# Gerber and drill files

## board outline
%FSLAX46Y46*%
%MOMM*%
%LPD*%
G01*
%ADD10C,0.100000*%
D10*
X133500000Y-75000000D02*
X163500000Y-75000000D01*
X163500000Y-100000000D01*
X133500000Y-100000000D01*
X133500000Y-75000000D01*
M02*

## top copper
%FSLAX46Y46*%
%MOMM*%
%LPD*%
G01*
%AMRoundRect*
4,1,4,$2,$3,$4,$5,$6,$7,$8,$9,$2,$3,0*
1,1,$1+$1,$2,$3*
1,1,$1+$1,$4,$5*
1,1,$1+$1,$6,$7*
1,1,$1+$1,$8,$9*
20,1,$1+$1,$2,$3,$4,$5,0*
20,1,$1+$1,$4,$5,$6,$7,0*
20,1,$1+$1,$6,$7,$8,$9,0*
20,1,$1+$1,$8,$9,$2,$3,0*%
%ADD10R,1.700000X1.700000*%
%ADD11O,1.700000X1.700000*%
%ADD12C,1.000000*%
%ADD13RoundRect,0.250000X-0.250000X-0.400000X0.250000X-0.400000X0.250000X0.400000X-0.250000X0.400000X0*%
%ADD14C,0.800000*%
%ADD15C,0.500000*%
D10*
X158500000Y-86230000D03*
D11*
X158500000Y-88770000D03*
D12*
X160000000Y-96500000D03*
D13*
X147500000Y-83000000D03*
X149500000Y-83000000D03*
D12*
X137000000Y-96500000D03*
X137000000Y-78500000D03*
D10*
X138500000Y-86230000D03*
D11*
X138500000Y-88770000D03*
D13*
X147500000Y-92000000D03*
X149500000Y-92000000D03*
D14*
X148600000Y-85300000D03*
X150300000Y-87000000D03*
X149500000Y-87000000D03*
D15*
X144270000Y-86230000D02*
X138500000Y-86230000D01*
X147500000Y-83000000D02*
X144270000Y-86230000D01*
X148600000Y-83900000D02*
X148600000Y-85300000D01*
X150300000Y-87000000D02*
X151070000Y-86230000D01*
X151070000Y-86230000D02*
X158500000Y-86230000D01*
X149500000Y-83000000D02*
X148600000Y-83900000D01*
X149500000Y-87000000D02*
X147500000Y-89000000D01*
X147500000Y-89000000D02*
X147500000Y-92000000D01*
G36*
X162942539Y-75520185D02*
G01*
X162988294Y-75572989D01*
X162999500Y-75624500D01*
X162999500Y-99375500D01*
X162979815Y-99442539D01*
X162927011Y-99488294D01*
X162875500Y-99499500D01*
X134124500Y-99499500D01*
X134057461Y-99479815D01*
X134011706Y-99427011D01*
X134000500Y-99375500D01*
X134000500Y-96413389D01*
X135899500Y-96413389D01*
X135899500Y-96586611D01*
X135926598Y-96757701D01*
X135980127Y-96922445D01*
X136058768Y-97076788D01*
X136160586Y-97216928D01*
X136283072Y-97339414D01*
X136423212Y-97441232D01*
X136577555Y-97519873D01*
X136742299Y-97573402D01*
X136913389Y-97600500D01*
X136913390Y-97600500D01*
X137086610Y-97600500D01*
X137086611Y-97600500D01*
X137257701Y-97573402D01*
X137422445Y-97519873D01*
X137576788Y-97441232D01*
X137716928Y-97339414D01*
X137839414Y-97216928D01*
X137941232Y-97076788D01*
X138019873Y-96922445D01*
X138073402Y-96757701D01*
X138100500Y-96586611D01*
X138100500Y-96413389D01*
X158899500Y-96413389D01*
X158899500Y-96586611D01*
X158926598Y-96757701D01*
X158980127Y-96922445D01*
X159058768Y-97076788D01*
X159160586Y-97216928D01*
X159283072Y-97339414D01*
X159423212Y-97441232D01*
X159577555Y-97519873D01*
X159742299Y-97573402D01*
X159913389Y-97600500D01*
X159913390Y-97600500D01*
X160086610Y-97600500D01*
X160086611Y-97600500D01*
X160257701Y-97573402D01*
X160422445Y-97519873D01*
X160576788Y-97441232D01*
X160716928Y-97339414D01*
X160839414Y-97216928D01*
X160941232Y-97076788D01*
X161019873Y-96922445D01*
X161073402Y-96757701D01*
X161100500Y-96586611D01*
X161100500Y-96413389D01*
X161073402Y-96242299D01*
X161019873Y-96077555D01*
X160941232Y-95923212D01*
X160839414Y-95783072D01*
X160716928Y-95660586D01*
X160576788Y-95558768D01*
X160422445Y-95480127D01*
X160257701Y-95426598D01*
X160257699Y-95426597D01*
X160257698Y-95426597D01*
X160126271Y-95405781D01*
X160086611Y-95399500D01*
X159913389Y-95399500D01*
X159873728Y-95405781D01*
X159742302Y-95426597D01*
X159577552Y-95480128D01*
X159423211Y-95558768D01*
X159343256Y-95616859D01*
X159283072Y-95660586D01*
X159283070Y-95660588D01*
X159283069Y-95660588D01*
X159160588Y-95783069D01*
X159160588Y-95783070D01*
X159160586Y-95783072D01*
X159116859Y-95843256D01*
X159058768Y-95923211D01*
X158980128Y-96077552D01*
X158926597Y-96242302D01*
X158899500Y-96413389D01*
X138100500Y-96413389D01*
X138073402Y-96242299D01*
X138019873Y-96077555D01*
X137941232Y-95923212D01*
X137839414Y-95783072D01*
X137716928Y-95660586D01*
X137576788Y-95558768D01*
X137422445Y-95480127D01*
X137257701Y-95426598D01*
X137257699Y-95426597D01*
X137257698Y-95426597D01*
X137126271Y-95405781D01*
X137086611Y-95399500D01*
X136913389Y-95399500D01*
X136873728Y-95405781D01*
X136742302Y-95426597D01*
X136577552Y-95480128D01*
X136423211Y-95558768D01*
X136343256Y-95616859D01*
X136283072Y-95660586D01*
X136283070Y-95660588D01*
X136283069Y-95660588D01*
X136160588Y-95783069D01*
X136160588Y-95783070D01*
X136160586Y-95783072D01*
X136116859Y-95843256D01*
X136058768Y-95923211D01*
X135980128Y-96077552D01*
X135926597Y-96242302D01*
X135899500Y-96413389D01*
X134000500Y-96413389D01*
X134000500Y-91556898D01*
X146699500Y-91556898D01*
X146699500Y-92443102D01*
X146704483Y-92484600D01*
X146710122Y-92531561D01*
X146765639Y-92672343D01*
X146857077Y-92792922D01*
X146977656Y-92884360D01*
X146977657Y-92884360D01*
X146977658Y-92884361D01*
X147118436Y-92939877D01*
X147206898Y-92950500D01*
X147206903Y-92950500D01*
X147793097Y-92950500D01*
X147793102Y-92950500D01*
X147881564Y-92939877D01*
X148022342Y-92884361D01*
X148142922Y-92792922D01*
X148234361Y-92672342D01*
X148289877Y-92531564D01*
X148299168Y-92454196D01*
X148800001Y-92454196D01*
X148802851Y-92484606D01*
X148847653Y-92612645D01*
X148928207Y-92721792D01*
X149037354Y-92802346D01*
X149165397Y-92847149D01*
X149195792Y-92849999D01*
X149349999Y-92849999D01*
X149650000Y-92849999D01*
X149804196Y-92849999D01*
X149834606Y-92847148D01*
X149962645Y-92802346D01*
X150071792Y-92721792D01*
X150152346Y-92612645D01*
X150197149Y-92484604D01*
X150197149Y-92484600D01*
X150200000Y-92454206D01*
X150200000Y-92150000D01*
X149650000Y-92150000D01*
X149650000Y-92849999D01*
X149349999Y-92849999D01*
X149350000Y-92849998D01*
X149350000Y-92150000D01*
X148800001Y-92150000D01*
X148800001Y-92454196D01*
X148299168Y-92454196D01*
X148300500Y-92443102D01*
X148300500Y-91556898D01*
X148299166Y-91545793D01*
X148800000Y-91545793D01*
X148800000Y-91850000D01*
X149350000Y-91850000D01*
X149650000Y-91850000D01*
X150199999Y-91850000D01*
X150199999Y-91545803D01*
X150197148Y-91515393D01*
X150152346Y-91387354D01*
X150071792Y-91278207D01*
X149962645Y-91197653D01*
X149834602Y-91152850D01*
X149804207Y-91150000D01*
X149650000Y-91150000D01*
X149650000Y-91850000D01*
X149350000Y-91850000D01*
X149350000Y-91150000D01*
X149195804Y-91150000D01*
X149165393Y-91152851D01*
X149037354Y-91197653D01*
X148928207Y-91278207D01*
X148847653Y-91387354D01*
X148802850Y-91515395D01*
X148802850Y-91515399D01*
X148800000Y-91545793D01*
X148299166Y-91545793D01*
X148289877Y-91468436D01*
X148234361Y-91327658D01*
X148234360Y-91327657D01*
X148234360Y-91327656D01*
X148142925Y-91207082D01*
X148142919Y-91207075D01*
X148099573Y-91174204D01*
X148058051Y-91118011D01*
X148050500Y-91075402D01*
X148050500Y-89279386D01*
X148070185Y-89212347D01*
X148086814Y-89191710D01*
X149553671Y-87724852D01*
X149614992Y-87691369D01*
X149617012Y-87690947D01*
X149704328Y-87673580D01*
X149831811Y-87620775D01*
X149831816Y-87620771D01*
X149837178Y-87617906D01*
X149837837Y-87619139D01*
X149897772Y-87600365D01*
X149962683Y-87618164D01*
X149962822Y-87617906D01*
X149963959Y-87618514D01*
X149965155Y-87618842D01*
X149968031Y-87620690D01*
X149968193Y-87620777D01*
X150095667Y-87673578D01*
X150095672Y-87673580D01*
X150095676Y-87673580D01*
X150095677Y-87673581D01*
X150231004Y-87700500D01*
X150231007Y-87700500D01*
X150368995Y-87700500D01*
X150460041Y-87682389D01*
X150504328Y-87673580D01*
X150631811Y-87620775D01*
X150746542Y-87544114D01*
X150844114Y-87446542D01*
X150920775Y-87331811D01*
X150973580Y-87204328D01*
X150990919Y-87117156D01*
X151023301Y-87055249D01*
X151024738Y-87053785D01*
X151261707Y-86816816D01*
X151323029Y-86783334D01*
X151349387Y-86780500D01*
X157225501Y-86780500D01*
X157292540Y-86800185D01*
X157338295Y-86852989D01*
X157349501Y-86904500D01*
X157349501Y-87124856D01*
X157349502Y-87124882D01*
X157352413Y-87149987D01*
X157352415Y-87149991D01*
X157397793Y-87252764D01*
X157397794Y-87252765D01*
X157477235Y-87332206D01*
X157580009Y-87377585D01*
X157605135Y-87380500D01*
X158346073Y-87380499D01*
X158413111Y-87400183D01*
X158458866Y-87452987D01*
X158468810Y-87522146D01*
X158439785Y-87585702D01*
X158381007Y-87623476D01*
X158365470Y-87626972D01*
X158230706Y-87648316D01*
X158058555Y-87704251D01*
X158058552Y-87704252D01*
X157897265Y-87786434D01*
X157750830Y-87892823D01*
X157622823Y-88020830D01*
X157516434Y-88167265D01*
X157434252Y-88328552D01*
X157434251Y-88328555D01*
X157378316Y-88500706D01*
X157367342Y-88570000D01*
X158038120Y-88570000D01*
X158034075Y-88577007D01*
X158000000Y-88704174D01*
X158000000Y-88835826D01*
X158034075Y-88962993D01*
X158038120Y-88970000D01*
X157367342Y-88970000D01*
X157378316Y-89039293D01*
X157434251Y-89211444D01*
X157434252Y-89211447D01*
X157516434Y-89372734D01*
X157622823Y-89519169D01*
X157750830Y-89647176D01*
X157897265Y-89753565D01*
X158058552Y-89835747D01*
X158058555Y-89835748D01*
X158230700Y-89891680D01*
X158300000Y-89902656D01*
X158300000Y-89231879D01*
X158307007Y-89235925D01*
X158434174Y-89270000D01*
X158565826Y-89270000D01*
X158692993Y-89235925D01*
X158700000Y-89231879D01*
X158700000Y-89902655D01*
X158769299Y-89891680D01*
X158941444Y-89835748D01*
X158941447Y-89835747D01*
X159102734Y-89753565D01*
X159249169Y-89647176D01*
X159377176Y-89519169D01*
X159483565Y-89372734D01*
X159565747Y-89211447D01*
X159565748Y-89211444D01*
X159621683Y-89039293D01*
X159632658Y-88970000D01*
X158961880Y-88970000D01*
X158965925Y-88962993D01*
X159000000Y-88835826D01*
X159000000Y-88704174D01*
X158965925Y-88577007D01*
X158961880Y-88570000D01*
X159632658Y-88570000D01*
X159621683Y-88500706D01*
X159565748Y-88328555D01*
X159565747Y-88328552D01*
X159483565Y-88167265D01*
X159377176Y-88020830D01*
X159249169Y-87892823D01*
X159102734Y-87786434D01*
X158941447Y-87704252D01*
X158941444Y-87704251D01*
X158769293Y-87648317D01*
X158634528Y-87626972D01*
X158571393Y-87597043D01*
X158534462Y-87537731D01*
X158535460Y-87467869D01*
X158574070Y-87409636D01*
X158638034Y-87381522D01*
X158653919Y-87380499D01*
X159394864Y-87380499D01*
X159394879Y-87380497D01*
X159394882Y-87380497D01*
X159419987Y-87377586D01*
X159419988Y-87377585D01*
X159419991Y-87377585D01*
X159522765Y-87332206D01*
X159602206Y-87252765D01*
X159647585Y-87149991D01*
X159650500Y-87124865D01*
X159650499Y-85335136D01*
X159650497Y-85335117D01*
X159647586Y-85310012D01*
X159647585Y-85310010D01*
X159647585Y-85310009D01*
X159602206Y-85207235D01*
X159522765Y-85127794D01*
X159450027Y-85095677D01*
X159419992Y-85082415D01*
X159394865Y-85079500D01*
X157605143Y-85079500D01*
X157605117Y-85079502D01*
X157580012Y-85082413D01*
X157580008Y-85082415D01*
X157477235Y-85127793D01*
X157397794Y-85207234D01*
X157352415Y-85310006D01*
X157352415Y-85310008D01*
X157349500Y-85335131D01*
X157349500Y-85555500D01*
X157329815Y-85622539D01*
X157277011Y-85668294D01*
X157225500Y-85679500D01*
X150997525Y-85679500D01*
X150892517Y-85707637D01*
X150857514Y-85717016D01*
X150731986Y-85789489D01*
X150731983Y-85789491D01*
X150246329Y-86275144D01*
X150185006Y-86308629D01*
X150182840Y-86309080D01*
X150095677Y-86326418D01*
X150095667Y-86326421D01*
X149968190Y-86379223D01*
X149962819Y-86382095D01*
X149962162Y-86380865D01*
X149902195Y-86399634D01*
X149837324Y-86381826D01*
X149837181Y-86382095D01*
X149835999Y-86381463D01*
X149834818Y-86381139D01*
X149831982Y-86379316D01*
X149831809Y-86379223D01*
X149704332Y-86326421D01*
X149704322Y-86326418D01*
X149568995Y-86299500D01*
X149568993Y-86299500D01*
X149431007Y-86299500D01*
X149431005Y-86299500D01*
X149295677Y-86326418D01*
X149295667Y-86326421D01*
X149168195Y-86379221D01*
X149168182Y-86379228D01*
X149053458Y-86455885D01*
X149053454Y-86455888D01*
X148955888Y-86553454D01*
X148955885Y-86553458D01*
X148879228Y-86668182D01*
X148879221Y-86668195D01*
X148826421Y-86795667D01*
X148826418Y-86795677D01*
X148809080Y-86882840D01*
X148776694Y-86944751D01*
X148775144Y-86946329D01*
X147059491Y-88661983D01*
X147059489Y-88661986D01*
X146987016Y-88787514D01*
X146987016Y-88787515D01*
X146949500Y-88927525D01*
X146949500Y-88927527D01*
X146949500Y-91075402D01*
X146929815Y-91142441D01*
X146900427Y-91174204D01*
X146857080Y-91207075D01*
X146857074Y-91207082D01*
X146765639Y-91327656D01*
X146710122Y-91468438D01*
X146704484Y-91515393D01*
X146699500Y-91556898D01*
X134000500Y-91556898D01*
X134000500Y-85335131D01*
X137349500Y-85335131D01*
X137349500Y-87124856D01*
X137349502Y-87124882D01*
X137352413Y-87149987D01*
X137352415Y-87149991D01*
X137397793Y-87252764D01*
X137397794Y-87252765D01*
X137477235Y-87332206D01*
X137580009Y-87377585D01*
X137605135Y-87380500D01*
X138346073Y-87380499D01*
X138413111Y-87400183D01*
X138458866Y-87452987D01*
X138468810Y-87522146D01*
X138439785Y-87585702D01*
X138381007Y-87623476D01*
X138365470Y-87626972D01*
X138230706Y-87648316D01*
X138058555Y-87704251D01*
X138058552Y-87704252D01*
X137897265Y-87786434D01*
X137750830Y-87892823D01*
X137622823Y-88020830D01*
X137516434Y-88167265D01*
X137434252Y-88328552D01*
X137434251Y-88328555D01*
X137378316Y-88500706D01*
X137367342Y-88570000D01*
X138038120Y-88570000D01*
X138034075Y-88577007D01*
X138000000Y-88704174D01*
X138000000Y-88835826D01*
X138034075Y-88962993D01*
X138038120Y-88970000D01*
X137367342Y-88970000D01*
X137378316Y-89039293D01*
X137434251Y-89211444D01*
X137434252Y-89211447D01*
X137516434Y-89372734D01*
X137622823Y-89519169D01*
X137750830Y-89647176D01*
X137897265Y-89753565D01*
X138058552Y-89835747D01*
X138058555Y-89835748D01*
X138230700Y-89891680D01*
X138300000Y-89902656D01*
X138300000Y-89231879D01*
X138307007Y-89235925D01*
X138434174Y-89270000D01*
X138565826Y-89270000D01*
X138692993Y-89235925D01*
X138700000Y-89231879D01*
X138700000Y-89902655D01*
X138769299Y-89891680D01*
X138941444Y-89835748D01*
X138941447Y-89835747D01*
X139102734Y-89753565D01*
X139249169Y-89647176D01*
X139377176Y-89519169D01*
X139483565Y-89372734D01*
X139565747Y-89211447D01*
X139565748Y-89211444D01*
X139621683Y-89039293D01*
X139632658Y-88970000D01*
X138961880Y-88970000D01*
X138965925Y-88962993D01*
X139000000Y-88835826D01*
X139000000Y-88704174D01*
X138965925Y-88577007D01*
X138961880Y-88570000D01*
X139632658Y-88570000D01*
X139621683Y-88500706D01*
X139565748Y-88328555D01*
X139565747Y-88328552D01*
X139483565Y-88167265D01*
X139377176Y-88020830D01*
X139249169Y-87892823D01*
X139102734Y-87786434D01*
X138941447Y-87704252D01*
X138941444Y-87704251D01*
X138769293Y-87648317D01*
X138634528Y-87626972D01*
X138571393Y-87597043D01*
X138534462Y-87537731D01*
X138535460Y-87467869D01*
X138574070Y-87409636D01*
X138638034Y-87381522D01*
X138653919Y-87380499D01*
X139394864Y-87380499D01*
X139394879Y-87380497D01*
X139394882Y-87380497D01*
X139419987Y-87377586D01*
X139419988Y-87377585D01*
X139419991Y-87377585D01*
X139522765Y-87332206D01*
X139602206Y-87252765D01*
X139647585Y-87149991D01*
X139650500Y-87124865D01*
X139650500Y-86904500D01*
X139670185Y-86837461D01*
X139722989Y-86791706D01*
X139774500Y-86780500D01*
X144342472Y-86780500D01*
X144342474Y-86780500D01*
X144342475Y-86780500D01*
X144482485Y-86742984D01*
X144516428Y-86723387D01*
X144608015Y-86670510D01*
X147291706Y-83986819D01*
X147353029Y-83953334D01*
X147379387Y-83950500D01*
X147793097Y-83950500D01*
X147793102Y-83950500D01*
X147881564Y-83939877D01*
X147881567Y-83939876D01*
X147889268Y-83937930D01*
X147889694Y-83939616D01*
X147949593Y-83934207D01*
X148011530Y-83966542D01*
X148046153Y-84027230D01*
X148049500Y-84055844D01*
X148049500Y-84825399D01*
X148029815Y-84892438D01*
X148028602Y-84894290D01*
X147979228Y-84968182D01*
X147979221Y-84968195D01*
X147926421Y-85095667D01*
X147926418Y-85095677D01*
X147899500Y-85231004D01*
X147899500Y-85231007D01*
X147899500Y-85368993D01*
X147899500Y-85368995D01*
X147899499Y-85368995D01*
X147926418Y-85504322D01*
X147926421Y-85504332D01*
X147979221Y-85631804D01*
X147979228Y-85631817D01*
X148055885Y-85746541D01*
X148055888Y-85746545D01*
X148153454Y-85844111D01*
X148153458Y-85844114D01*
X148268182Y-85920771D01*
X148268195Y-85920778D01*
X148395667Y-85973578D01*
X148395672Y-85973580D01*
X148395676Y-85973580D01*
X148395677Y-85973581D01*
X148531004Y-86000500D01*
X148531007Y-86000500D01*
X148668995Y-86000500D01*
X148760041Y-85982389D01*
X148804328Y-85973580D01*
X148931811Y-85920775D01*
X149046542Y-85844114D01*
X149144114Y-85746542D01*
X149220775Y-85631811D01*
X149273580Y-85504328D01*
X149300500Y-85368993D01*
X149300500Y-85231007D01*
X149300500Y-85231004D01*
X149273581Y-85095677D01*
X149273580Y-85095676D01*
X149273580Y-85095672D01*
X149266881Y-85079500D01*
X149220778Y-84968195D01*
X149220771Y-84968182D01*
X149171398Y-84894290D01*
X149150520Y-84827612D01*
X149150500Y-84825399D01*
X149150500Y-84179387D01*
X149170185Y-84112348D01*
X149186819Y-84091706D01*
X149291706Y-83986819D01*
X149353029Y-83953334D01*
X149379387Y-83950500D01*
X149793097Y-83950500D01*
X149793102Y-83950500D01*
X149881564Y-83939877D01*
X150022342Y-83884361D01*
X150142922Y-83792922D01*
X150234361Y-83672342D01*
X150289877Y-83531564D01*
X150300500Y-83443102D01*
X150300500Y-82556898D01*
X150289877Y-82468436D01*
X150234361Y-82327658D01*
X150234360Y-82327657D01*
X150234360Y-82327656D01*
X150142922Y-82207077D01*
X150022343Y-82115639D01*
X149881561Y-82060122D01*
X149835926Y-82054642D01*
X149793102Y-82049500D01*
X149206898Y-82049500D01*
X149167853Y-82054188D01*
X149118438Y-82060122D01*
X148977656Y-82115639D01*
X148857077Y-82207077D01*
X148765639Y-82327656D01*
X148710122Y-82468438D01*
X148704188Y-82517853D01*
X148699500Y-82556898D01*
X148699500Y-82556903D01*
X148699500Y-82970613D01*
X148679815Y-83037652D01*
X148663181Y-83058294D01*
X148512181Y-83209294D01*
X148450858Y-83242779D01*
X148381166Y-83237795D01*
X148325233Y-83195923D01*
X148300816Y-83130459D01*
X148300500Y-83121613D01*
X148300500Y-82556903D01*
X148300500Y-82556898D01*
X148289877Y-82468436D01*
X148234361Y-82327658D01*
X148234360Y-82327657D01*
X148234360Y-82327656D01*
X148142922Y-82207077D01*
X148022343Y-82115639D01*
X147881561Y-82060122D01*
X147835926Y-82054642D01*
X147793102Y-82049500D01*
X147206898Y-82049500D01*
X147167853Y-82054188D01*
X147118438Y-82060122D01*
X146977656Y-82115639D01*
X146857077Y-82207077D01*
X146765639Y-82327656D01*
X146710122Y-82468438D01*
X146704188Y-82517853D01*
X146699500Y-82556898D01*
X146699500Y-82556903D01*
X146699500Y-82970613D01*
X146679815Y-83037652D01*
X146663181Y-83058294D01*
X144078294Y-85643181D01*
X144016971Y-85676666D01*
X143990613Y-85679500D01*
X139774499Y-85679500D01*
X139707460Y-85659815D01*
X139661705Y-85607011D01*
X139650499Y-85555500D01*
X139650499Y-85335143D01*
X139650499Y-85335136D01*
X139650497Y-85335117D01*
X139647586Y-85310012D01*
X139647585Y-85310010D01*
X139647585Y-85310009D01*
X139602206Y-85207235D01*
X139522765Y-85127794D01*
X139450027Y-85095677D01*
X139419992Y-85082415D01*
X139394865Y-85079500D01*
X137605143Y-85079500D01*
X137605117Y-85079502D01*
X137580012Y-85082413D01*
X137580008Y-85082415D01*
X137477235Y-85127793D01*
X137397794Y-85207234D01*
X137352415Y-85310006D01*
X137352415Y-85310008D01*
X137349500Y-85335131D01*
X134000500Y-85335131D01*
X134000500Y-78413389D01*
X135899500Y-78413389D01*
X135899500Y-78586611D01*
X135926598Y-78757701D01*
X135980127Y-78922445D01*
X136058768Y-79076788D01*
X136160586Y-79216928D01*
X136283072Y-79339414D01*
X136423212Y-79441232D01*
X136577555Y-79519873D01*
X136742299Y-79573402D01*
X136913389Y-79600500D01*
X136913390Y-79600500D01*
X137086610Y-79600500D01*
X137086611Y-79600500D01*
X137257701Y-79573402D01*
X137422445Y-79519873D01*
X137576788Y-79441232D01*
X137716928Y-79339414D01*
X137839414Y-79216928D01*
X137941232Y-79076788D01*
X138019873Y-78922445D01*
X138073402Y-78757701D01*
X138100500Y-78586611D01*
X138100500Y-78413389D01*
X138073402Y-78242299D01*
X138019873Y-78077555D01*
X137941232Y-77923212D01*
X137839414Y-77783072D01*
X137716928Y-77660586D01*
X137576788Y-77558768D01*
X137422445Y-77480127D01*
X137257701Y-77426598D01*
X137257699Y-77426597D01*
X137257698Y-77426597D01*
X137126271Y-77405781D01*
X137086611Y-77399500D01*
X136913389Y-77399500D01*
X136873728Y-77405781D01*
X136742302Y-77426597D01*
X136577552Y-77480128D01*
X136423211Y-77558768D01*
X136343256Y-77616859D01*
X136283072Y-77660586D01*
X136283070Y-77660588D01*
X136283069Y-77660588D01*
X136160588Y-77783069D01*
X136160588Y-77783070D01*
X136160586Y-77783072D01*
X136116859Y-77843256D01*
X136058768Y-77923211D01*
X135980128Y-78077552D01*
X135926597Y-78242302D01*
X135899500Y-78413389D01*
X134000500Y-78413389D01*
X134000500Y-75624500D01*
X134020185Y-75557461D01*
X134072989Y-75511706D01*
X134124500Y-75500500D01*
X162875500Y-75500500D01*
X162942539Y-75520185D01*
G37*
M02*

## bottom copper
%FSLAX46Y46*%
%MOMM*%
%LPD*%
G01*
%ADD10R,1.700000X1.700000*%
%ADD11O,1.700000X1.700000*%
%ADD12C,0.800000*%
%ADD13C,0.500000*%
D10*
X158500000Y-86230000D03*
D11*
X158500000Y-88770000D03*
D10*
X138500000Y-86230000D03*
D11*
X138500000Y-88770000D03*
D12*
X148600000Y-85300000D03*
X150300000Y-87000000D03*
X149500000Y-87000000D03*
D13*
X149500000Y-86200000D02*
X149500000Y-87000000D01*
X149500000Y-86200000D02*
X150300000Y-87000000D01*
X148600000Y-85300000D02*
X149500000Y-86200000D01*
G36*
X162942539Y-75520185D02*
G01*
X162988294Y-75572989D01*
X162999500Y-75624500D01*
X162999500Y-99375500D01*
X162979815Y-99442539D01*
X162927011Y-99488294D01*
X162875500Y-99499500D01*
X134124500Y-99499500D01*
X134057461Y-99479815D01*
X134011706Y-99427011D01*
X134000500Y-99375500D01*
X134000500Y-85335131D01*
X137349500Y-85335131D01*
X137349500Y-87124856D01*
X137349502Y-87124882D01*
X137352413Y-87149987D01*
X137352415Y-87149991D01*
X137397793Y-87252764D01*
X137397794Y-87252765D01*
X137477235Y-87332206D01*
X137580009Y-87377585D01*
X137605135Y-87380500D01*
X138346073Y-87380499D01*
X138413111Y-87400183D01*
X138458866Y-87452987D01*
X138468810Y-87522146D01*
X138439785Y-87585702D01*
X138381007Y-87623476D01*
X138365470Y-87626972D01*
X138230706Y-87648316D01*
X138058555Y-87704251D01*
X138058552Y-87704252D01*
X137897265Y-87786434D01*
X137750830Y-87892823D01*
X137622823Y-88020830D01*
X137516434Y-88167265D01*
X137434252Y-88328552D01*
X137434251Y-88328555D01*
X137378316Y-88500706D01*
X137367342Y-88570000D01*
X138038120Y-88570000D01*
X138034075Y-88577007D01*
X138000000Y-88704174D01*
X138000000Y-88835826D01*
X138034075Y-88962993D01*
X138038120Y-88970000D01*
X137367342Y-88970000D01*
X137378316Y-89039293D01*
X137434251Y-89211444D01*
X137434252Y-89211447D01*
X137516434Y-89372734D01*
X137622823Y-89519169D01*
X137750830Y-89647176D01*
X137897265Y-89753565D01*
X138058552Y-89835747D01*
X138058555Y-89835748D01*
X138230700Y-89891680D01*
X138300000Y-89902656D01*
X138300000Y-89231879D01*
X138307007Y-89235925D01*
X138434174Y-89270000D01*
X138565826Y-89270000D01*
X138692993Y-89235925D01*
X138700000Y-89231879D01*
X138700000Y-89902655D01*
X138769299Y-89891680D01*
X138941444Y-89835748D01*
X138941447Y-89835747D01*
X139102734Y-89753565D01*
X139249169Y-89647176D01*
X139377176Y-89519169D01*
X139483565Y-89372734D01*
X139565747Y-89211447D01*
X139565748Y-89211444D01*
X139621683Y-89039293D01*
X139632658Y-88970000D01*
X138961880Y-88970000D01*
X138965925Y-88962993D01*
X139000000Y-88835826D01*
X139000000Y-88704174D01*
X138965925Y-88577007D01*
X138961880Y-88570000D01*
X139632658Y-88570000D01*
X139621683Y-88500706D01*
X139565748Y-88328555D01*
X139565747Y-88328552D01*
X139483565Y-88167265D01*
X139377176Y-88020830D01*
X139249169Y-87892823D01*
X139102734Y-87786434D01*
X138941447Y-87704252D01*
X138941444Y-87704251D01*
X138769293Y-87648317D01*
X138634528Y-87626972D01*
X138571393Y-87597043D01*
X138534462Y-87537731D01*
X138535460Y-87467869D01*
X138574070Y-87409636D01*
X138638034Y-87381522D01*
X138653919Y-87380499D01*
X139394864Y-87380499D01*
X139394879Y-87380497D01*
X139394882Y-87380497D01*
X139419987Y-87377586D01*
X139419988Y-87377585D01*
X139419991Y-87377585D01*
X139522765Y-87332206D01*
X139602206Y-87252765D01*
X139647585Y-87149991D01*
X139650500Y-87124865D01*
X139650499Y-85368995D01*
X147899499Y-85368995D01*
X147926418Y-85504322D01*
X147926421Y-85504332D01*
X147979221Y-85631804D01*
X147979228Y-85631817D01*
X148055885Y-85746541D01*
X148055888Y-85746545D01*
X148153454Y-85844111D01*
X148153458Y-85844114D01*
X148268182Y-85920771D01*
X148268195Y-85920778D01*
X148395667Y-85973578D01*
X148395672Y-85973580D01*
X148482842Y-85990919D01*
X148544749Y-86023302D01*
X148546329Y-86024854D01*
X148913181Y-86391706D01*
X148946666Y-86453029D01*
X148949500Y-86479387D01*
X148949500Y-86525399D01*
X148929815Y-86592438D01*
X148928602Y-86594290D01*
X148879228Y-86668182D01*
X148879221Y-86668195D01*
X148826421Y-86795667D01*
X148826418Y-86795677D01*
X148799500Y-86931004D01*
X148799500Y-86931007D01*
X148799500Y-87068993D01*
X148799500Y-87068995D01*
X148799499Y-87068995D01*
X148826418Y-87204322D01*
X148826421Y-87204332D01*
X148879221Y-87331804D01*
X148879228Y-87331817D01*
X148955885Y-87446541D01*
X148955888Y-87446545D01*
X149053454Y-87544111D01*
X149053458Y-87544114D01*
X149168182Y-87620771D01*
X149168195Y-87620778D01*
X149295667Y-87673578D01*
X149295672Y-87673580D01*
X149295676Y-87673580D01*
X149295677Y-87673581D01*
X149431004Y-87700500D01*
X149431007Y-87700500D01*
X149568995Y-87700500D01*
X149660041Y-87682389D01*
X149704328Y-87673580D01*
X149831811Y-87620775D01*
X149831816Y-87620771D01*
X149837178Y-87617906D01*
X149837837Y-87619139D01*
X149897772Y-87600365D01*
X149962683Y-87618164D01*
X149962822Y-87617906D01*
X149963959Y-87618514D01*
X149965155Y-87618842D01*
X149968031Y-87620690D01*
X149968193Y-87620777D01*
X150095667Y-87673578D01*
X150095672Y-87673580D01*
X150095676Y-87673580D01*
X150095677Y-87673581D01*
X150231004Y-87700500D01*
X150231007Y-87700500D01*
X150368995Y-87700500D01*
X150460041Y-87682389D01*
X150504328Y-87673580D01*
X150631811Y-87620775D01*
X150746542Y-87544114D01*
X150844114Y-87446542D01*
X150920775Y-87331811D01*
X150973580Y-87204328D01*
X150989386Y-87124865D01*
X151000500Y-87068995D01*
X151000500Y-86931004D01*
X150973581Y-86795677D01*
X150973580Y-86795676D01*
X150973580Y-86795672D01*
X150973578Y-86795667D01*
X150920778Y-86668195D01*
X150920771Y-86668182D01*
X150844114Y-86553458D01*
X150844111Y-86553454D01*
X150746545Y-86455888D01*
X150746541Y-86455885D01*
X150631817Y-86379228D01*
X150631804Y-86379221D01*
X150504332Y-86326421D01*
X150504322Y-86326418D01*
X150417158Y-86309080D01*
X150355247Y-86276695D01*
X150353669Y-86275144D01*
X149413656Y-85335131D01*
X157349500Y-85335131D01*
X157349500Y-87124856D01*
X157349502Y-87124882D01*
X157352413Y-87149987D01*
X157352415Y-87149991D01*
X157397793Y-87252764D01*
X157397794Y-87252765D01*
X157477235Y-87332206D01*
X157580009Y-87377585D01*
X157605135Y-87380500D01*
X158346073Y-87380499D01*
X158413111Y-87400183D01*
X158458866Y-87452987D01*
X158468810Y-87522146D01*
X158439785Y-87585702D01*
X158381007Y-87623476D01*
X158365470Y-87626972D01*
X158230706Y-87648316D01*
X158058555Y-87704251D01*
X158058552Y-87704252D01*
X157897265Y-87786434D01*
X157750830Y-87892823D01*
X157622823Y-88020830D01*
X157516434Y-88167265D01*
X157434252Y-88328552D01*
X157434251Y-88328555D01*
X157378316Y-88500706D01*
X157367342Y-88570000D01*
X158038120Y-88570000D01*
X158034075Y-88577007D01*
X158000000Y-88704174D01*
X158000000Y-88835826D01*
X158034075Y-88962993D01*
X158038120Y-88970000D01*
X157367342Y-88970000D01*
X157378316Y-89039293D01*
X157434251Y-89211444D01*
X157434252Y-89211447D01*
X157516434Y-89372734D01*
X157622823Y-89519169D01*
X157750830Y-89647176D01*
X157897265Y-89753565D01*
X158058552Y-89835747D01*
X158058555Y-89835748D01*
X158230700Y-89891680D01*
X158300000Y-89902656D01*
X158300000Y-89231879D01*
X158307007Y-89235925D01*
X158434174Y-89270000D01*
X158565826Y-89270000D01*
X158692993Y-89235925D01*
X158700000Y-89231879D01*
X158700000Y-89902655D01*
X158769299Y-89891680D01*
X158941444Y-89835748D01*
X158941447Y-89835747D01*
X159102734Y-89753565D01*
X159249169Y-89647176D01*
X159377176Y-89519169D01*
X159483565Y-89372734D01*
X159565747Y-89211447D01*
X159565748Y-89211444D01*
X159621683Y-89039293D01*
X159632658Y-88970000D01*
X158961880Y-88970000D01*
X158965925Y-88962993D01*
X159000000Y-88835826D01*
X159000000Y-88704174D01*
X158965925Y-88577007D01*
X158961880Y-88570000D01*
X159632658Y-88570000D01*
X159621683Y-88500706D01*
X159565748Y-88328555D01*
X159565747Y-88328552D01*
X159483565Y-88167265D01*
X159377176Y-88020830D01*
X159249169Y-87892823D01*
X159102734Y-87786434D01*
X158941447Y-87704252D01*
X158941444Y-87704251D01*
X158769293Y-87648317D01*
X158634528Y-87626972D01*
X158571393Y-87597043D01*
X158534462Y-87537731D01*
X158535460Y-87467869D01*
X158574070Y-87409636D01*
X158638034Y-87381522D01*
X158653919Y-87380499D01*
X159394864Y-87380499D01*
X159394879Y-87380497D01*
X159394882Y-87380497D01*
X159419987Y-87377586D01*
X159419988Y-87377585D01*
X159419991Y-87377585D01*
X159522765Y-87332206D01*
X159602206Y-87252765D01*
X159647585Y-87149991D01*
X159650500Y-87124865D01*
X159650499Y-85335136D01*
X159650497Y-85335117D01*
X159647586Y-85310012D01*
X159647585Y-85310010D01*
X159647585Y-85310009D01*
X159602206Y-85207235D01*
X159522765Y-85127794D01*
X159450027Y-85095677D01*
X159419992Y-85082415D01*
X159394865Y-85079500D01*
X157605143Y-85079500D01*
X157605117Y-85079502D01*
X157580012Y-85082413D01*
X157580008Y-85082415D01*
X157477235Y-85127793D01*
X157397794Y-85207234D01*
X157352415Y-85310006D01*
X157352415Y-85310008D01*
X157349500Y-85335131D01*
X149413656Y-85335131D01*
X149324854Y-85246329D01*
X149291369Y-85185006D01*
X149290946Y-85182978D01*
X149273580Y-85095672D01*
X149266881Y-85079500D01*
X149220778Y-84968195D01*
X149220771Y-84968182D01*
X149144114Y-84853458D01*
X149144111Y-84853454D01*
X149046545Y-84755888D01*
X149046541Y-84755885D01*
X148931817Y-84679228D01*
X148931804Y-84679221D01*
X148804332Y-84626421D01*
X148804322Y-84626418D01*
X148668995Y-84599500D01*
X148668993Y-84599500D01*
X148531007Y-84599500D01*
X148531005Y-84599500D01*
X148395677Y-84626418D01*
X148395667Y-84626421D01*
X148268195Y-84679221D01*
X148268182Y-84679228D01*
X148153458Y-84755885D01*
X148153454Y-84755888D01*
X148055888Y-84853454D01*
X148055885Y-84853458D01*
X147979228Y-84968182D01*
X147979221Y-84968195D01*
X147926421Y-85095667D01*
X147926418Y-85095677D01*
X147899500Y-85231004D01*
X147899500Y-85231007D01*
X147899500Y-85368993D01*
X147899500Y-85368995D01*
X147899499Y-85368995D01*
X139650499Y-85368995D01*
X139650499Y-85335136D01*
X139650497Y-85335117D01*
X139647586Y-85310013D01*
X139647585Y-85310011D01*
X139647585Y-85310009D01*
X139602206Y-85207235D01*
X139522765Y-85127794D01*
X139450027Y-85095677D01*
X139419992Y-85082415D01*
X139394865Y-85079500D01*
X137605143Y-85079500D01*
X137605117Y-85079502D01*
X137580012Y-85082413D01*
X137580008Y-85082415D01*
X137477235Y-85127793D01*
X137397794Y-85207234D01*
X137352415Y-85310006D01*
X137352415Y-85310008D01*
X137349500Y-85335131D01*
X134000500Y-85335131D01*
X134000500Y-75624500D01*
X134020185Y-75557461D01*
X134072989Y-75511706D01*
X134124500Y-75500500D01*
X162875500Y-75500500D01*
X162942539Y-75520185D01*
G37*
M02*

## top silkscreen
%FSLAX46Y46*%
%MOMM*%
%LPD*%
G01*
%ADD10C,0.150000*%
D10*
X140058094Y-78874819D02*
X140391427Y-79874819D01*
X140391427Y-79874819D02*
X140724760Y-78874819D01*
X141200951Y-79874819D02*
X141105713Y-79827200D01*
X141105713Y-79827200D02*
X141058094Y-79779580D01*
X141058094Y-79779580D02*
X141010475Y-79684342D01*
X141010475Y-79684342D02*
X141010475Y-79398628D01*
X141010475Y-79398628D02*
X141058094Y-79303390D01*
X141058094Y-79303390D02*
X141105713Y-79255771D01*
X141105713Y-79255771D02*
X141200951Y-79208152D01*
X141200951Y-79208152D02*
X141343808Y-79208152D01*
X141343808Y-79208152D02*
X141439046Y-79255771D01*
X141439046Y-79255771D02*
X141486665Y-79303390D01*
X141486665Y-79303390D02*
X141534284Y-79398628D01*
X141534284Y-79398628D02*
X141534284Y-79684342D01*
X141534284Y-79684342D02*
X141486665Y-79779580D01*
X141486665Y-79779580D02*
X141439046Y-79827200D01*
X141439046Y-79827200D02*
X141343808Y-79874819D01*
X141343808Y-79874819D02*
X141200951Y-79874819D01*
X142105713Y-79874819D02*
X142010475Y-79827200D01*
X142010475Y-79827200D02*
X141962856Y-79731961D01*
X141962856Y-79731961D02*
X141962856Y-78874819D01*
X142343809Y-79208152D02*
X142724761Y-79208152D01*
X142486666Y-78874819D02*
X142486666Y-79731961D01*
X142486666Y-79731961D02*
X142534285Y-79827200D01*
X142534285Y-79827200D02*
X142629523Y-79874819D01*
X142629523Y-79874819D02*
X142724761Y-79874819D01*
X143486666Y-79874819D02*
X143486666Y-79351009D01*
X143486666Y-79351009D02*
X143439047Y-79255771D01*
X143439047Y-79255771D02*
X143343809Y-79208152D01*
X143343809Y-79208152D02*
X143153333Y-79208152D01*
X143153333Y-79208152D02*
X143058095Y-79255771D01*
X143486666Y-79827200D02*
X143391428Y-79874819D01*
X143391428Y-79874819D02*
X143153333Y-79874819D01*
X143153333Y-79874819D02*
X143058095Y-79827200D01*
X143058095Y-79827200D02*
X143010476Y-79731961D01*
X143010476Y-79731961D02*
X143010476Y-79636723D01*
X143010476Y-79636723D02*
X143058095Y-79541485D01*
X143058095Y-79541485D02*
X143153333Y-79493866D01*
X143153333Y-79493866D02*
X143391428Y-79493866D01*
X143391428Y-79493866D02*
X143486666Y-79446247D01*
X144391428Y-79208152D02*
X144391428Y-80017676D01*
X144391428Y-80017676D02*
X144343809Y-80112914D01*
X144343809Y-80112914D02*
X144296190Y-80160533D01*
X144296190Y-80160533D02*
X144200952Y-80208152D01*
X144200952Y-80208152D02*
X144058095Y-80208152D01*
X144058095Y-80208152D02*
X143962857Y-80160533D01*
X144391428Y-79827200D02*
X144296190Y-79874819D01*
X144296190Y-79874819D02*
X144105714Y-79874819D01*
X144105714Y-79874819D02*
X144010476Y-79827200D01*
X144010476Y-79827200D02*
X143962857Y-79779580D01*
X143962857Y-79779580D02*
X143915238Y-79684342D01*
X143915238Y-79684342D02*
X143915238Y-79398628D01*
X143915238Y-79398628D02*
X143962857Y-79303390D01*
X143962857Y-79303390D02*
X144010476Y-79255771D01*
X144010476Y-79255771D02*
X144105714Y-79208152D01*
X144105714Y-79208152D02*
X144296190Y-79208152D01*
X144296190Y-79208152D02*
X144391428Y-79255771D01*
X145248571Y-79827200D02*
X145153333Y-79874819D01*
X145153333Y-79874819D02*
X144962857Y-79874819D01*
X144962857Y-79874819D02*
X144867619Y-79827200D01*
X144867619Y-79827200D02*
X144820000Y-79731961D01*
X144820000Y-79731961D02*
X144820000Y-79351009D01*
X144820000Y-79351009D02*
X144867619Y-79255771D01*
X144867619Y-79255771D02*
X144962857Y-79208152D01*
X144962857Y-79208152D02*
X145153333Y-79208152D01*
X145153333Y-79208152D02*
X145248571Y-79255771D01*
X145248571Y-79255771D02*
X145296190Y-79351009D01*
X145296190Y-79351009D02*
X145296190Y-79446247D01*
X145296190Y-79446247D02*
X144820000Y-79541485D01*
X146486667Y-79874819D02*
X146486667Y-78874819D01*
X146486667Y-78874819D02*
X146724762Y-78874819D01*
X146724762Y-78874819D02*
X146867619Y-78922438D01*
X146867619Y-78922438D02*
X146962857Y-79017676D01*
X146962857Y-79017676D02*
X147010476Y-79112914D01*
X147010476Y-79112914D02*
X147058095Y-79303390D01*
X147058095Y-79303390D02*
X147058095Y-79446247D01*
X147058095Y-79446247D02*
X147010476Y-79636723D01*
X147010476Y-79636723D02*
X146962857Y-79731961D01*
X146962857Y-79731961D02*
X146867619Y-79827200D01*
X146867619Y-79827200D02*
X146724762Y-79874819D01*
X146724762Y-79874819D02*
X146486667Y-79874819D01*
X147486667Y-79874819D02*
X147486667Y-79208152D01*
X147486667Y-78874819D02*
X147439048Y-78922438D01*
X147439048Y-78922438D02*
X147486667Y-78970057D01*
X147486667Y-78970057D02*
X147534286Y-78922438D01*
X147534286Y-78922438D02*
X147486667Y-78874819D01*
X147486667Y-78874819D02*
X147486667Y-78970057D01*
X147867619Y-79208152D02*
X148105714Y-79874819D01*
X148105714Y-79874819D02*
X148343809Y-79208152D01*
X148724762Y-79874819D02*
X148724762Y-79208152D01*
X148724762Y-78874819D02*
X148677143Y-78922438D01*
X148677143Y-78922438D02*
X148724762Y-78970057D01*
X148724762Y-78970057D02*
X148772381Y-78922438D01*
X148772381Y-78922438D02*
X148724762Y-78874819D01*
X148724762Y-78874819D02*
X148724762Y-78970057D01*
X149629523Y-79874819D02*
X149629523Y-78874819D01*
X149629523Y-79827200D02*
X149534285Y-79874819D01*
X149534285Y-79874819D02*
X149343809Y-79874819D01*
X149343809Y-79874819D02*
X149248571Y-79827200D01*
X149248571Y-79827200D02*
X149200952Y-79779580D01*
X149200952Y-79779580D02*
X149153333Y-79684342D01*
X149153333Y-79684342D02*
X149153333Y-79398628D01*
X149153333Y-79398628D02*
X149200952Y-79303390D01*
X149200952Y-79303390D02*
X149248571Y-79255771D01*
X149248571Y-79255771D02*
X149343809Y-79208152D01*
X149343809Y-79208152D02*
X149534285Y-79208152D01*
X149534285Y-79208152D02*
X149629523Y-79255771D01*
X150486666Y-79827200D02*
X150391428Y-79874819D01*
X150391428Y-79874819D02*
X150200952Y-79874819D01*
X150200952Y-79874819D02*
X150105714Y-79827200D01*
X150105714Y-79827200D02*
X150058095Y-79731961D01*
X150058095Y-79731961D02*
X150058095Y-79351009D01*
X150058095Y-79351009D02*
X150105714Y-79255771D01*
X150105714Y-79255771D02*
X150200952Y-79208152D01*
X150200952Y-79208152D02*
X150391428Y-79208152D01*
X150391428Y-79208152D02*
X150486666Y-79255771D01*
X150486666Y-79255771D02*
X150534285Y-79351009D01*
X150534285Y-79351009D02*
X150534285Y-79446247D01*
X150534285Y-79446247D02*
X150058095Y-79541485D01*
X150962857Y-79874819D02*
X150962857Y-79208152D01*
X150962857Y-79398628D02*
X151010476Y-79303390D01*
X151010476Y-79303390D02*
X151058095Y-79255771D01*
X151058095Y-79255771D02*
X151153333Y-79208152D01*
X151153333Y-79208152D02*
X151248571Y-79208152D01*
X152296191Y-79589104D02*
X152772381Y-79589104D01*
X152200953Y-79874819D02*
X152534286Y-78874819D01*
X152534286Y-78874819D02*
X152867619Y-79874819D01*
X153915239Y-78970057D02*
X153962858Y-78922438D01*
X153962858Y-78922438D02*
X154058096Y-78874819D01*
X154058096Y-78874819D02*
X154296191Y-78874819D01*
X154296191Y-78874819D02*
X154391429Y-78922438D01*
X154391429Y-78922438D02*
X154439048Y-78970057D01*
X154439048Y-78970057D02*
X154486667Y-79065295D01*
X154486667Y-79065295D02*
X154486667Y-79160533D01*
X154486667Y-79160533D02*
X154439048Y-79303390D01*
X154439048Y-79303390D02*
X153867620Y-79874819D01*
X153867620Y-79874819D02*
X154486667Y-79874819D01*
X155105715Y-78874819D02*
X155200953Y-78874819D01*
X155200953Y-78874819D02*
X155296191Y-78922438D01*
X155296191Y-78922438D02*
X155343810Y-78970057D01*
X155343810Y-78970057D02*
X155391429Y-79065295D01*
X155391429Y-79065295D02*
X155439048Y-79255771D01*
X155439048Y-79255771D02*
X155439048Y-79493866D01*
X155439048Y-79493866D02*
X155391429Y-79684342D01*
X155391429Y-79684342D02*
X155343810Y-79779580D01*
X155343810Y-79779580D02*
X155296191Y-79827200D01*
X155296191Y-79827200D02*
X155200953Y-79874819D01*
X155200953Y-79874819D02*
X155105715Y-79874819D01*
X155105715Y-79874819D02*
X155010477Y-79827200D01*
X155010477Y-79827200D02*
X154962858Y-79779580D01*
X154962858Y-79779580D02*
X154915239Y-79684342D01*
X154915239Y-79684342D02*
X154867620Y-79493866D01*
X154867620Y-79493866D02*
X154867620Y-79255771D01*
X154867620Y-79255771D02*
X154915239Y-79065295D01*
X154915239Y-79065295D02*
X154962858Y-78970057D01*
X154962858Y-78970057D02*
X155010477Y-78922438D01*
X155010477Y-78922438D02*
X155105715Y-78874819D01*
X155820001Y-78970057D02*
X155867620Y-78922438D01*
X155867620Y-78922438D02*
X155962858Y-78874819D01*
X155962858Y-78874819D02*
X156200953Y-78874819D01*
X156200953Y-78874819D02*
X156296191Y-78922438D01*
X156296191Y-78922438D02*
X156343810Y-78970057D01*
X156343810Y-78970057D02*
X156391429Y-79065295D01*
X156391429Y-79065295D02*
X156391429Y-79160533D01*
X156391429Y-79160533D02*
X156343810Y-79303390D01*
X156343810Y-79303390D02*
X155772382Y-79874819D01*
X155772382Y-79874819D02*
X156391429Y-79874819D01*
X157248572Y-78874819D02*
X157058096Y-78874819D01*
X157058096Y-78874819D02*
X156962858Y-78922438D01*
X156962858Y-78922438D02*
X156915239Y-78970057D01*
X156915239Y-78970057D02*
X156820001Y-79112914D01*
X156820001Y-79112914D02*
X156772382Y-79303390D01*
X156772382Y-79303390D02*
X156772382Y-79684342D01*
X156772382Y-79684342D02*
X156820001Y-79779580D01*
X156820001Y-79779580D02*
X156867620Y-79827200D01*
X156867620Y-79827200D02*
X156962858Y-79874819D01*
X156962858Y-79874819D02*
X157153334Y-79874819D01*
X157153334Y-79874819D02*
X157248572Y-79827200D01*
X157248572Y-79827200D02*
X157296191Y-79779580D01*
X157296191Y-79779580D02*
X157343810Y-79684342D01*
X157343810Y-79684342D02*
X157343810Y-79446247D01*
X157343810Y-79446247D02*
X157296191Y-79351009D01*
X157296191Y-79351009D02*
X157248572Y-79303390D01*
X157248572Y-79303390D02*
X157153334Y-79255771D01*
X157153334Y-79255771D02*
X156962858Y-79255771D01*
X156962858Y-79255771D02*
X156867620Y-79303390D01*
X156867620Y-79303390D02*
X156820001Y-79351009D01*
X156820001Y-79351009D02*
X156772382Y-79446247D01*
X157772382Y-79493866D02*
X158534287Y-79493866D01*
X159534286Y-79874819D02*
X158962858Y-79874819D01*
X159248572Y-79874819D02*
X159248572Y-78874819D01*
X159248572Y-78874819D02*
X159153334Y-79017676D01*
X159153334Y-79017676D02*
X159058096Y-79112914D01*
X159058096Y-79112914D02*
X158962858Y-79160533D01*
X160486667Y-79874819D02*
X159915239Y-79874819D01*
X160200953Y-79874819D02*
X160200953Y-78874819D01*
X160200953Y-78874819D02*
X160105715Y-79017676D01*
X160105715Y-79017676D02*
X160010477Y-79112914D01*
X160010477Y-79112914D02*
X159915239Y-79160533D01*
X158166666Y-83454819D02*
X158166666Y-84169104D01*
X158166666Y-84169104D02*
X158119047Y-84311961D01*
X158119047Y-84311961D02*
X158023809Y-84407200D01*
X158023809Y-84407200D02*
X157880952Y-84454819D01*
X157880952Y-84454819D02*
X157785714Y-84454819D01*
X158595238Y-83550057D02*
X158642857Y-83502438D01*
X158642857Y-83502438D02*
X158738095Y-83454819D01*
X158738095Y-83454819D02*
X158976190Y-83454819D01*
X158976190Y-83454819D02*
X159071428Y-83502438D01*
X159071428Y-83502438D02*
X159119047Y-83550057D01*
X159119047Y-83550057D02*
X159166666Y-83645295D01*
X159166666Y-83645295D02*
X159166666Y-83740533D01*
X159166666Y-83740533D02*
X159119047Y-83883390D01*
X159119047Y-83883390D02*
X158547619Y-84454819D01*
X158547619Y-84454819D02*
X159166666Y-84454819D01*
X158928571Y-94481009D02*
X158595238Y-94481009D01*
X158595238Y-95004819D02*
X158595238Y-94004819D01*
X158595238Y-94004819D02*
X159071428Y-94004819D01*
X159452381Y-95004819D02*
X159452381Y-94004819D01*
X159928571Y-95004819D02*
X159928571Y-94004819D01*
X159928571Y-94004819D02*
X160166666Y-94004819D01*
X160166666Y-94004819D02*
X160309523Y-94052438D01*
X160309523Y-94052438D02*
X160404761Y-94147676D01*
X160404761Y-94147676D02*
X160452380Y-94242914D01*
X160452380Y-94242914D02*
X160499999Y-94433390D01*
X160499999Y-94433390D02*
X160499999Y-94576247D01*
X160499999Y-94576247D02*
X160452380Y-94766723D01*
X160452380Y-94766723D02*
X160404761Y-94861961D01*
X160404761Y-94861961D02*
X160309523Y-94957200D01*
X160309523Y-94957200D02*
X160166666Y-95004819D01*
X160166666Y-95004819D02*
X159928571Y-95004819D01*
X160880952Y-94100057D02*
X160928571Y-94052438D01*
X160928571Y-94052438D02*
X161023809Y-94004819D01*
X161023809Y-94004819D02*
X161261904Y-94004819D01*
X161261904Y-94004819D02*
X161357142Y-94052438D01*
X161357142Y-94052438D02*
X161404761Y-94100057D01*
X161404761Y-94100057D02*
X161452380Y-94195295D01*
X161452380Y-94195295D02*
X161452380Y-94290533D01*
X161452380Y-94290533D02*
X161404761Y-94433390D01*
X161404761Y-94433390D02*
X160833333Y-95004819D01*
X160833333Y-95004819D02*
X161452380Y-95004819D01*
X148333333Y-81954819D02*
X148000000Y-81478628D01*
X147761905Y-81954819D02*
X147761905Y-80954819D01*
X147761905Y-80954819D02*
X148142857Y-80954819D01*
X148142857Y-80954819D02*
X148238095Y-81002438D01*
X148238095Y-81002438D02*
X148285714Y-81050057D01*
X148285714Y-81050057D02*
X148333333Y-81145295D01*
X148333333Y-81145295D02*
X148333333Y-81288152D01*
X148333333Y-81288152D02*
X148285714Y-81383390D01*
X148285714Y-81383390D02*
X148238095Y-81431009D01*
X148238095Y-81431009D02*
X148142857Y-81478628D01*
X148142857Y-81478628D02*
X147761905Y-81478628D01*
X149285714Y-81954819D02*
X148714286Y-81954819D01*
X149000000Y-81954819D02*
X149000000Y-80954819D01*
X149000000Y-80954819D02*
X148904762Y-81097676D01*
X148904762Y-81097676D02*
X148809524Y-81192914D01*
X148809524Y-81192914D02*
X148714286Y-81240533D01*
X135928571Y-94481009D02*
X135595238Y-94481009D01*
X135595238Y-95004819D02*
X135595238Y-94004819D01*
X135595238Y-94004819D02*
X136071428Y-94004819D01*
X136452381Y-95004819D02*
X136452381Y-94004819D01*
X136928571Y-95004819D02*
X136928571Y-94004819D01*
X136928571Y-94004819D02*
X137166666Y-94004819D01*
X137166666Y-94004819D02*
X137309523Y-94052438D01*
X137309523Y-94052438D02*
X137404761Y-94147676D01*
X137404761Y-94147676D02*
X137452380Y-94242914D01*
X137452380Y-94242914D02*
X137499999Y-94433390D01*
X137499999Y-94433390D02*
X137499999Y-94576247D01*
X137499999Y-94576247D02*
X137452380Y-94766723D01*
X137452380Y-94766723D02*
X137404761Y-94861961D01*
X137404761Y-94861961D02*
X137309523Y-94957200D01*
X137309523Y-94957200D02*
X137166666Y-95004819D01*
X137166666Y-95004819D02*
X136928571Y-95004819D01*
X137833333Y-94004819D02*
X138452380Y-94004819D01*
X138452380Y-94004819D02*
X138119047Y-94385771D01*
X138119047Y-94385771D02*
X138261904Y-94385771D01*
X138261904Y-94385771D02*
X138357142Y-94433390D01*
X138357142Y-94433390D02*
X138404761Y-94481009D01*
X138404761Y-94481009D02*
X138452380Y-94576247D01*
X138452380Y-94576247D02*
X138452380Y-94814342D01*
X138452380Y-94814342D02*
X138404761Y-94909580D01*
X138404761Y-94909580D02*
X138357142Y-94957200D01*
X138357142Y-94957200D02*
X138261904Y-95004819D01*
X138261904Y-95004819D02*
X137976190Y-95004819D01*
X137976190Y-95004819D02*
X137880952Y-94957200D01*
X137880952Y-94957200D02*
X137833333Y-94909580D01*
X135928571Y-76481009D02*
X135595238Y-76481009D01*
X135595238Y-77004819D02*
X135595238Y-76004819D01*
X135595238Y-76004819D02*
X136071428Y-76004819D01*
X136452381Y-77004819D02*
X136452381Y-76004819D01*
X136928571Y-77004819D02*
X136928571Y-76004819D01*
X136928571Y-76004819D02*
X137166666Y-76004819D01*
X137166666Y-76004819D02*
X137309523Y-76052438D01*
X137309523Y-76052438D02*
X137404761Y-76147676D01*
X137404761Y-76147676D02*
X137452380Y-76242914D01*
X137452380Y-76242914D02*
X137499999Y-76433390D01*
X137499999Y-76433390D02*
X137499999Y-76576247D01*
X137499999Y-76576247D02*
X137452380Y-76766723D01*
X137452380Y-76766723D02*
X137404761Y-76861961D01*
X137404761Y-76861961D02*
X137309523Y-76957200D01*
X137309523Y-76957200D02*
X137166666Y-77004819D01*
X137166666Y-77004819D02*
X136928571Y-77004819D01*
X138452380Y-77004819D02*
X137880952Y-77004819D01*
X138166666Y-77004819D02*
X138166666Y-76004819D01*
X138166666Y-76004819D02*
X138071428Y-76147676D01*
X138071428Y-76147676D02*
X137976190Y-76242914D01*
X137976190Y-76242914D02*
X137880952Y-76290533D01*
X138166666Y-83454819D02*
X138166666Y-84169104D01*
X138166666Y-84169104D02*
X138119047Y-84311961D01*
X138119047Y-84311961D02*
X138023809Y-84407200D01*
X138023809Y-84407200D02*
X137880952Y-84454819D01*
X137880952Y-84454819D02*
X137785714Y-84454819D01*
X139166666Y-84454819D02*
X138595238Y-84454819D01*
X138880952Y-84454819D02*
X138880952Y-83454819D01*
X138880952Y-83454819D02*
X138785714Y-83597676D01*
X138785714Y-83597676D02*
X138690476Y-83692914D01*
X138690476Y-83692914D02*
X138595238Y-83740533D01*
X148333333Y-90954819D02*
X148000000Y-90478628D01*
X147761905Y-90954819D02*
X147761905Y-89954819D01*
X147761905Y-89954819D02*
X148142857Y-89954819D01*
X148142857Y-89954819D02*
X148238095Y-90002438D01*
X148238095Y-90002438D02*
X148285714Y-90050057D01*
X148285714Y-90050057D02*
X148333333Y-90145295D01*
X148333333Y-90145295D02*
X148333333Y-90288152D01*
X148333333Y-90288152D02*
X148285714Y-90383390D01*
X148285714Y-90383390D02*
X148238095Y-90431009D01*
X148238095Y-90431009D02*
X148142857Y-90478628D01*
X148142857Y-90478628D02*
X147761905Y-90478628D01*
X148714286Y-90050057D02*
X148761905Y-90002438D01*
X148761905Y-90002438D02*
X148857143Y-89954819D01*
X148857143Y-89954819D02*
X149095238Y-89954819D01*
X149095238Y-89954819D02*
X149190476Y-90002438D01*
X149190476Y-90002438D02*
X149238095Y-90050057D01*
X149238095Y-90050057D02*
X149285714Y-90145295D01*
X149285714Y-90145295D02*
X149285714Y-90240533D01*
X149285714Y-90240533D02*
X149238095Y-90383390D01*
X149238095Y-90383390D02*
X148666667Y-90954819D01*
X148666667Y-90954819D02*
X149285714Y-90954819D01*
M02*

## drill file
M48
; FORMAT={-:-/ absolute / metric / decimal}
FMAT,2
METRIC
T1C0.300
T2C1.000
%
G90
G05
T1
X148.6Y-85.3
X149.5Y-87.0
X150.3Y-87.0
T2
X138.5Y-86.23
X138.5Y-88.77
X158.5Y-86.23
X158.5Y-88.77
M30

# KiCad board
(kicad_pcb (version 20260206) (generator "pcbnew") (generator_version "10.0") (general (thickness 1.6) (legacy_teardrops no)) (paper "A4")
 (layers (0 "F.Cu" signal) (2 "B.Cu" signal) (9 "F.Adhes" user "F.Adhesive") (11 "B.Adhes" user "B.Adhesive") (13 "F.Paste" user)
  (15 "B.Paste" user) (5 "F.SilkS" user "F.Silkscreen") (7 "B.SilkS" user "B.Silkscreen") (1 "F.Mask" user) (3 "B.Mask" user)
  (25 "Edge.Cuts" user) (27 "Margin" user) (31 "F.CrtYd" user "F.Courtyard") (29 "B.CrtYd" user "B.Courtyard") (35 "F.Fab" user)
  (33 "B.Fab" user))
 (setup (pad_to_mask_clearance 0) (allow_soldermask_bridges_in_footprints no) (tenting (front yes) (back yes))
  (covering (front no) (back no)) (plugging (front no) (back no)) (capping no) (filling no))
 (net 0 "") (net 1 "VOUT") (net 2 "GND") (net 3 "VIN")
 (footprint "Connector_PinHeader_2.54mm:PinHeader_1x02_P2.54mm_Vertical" (layer "F.Cu") (at 158.5 87.5)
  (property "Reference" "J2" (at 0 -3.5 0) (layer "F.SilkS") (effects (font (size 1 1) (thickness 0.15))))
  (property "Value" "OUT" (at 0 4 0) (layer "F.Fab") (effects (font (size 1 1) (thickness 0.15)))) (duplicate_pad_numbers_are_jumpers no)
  (pad "1" thru_hole rect (at 0 -1.27) (size 1.7 1.7) (drill 1) (layers "*.Cu" "*.Mask") (remove_unused_layers no) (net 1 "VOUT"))
  (pad "2" thru_hole oval (at 0 1.27) (size 1.7 1.7) (drill 1) (layers "*.Cu" "*.Mask") (remove_unused_layers no) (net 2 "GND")))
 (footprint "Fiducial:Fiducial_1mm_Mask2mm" (layer "F.Cu") (at 160 96.5)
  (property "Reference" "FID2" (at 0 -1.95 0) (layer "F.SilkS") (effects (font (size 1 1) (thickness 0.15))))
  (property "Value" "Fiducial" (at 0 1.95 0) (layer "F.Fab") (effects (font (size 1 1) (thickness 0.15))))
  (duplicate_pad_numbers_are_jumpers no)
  (pad "" smd circle (at 0 0) (size 1 1) (layers "F.Cu" "F.Mask") (solder_mask_margin 0.5) (clearance 0.6)))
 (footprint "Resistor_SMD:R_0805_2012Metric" (layer "F.Cu") (at 148.5 83)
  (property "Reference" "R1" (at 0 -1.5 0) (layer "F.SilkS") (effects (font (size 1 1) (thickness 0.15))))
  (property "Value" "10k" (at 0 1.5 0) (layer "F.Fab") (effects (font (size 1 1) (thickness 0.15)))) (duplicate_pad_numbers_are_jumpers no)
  (pad "1" smd roundrect (at -1 0) (size 1 1.3) (layers "F.Cu" "F.Mask" "F.Paste") (roundrect_rratio 0.25) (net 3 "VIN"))
  (pad "2" smd roundrect (at 1 0) (size 1 1.3) (layers "F.Cu" "F.Mask" "F.Paste") (roundrect_rratio 0.25) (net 1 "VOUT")))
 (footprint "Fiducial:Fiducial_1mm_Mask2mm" (layer "F.Cu") (at 137 96.5)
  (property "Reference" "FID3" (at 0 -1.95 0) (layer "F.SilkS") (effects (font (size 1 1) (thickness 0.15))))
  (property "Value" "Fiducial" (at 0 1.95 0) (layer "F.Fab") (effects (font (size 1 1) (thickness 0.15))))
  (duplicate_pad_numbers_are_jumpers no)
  (pad "" smd circle (at 0 0) (size 1 1) (layers "F.Cu" "F.Mask") (solder_mask_margin 0.5) (clearance 0.6)))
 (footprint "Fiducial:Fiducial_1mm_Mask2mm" (layer "F.Cu") (at 137 78.5)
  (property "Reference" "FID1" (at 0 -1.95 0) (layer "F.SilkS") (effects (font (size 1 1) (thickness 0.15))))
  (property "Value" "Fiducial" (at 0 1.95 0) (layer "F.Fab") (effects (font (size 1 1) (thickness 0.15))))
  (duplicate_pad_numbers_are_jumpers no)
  (pad "" smd circle (at 0 0) (size 1 1) (layers "F.Cu" "F.Mask") (solder_mask_margin 0.5) (clearance 0.6)))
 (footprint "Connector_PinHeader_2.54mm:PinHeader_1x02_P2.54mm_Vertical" (layer "F.Cu") (at 138.5 87.5)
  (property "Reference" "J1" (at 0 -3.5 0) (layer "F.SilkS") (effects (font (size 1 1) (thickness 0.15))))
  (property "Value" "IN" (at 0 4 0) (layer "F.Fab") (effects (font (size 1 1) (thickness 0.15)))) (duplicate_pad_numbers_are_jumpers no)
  (pad "1" thru_hole rect (at 0 -1.27) (size 1.7 1.7) (drill 1) (layers "*.Cu" "*.Mask") (remove_unused_layers no) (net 3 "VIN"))
  (pad "2" thru_hole oval (at 0 1.27) (size 1.7 1.7) (drill 1) (layers "*.Cu" "*.Mask") (remove_unused_layers no) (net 2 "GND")))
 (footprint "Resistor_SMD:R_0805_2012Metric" (layer "F.Cu") (at 148.5 92)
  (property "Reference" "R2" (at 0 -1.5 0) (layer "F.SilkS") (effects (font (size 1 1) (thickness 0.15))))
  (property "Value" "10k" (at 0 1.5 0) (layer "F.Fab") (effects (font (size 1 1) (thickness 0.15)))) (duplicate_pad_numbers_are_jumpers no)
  (pad "1" smd roundrect (at -1 0) (size 1 1.3) (layers "F.Cu" "F.Mask" "F.Paste") (roundrect_rratio 0.25) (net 1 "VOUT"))
  (pad "2" smd roundrect (at 1 0) (size 1 1.3) (layers "F.Cu" "F.Mask" "F.Paste") (roundrect_rratio 0.25) (thermal_bridge_width 0.3)
   (thermal_gap 0.2) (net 2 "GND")))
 (gr_rect (start 133.5 75) (end 163.5 100) (stroke (width 0.1) (type default)) (fill no) (layer "Edge.Cuts"))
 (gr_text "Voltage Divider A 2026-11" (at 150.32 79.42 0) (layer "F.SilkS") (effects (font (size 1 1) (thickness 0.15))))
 (segment (start 144.27 86.23) (end 138.5 86.23) (width 0.5) (layer "F.Cu") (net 3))
 (segment (start 147.5 83) (end 144.27 86.23) (width 0.5) (layer "F.Cu") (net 3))
 (segment (start 148.6 83.9) (end 148.6 85.3) (width 0.5) (layer "F.Cu") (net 1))
 (segment (start 150.3 87) (end 151.07 86.23) (width 0.5) (layer "F.Cu") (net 1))
 (segment (start 151.07 86.23) (end 158.5 86.23) (width 0.5) (layer "F.Cu") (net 1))
 (segment (start 149.5 83) (end 148.6 83.9) (width 0.5) (layer "F.Cu") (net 1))
 (segment (start 149.5 87) (end 147.5 89) (width 0.5) (layer "F.Cu") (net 1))
 (segment (start 147.5 89) (end 147.5 92) (width 0.5) (layer "F.Cu") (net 1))
 (via (at 148.6 85.3) (size 0.8) (drill 0.3) (layers "F.Cu" "B.Cu") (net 1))
 (via (at 150.3 87) (size 0.8) (drill 0.3) (layers "F.Cu" "B.Cu") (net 1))
 (via (at 149.5 87) (size 0.8) (drill 0.3) (layers "F.Cu" "B.Cu") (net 1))
 (segment (start 149.5 86.2) (end 149.5 87) (width 0.5) (layer "B.Cu") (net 1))
 (segment (start 149.5 86.2) (end 150.3 87) (width 0.5) (layer "B.Cu") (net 1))
 (segment (start 148.6 85.3) (end 149.5 86.2) (width 0.5) (layer "B.Cu") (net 1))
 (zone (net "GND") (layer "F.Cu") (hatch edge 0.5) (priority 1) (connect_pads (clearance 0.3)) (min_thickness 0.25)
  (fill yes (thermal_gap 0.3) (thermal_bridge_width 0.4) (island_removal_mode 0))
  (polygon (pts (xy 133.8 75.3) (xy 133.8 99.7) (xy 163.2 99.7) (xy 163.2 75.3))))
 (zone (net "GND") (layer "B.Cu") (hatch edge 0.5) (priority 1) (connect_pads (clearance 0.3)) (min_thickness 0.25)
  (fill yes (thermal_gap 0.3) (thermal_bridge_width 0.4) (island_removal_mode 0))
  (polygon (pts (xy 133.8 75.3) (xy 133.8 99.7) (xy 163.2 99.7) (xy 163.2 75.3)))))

